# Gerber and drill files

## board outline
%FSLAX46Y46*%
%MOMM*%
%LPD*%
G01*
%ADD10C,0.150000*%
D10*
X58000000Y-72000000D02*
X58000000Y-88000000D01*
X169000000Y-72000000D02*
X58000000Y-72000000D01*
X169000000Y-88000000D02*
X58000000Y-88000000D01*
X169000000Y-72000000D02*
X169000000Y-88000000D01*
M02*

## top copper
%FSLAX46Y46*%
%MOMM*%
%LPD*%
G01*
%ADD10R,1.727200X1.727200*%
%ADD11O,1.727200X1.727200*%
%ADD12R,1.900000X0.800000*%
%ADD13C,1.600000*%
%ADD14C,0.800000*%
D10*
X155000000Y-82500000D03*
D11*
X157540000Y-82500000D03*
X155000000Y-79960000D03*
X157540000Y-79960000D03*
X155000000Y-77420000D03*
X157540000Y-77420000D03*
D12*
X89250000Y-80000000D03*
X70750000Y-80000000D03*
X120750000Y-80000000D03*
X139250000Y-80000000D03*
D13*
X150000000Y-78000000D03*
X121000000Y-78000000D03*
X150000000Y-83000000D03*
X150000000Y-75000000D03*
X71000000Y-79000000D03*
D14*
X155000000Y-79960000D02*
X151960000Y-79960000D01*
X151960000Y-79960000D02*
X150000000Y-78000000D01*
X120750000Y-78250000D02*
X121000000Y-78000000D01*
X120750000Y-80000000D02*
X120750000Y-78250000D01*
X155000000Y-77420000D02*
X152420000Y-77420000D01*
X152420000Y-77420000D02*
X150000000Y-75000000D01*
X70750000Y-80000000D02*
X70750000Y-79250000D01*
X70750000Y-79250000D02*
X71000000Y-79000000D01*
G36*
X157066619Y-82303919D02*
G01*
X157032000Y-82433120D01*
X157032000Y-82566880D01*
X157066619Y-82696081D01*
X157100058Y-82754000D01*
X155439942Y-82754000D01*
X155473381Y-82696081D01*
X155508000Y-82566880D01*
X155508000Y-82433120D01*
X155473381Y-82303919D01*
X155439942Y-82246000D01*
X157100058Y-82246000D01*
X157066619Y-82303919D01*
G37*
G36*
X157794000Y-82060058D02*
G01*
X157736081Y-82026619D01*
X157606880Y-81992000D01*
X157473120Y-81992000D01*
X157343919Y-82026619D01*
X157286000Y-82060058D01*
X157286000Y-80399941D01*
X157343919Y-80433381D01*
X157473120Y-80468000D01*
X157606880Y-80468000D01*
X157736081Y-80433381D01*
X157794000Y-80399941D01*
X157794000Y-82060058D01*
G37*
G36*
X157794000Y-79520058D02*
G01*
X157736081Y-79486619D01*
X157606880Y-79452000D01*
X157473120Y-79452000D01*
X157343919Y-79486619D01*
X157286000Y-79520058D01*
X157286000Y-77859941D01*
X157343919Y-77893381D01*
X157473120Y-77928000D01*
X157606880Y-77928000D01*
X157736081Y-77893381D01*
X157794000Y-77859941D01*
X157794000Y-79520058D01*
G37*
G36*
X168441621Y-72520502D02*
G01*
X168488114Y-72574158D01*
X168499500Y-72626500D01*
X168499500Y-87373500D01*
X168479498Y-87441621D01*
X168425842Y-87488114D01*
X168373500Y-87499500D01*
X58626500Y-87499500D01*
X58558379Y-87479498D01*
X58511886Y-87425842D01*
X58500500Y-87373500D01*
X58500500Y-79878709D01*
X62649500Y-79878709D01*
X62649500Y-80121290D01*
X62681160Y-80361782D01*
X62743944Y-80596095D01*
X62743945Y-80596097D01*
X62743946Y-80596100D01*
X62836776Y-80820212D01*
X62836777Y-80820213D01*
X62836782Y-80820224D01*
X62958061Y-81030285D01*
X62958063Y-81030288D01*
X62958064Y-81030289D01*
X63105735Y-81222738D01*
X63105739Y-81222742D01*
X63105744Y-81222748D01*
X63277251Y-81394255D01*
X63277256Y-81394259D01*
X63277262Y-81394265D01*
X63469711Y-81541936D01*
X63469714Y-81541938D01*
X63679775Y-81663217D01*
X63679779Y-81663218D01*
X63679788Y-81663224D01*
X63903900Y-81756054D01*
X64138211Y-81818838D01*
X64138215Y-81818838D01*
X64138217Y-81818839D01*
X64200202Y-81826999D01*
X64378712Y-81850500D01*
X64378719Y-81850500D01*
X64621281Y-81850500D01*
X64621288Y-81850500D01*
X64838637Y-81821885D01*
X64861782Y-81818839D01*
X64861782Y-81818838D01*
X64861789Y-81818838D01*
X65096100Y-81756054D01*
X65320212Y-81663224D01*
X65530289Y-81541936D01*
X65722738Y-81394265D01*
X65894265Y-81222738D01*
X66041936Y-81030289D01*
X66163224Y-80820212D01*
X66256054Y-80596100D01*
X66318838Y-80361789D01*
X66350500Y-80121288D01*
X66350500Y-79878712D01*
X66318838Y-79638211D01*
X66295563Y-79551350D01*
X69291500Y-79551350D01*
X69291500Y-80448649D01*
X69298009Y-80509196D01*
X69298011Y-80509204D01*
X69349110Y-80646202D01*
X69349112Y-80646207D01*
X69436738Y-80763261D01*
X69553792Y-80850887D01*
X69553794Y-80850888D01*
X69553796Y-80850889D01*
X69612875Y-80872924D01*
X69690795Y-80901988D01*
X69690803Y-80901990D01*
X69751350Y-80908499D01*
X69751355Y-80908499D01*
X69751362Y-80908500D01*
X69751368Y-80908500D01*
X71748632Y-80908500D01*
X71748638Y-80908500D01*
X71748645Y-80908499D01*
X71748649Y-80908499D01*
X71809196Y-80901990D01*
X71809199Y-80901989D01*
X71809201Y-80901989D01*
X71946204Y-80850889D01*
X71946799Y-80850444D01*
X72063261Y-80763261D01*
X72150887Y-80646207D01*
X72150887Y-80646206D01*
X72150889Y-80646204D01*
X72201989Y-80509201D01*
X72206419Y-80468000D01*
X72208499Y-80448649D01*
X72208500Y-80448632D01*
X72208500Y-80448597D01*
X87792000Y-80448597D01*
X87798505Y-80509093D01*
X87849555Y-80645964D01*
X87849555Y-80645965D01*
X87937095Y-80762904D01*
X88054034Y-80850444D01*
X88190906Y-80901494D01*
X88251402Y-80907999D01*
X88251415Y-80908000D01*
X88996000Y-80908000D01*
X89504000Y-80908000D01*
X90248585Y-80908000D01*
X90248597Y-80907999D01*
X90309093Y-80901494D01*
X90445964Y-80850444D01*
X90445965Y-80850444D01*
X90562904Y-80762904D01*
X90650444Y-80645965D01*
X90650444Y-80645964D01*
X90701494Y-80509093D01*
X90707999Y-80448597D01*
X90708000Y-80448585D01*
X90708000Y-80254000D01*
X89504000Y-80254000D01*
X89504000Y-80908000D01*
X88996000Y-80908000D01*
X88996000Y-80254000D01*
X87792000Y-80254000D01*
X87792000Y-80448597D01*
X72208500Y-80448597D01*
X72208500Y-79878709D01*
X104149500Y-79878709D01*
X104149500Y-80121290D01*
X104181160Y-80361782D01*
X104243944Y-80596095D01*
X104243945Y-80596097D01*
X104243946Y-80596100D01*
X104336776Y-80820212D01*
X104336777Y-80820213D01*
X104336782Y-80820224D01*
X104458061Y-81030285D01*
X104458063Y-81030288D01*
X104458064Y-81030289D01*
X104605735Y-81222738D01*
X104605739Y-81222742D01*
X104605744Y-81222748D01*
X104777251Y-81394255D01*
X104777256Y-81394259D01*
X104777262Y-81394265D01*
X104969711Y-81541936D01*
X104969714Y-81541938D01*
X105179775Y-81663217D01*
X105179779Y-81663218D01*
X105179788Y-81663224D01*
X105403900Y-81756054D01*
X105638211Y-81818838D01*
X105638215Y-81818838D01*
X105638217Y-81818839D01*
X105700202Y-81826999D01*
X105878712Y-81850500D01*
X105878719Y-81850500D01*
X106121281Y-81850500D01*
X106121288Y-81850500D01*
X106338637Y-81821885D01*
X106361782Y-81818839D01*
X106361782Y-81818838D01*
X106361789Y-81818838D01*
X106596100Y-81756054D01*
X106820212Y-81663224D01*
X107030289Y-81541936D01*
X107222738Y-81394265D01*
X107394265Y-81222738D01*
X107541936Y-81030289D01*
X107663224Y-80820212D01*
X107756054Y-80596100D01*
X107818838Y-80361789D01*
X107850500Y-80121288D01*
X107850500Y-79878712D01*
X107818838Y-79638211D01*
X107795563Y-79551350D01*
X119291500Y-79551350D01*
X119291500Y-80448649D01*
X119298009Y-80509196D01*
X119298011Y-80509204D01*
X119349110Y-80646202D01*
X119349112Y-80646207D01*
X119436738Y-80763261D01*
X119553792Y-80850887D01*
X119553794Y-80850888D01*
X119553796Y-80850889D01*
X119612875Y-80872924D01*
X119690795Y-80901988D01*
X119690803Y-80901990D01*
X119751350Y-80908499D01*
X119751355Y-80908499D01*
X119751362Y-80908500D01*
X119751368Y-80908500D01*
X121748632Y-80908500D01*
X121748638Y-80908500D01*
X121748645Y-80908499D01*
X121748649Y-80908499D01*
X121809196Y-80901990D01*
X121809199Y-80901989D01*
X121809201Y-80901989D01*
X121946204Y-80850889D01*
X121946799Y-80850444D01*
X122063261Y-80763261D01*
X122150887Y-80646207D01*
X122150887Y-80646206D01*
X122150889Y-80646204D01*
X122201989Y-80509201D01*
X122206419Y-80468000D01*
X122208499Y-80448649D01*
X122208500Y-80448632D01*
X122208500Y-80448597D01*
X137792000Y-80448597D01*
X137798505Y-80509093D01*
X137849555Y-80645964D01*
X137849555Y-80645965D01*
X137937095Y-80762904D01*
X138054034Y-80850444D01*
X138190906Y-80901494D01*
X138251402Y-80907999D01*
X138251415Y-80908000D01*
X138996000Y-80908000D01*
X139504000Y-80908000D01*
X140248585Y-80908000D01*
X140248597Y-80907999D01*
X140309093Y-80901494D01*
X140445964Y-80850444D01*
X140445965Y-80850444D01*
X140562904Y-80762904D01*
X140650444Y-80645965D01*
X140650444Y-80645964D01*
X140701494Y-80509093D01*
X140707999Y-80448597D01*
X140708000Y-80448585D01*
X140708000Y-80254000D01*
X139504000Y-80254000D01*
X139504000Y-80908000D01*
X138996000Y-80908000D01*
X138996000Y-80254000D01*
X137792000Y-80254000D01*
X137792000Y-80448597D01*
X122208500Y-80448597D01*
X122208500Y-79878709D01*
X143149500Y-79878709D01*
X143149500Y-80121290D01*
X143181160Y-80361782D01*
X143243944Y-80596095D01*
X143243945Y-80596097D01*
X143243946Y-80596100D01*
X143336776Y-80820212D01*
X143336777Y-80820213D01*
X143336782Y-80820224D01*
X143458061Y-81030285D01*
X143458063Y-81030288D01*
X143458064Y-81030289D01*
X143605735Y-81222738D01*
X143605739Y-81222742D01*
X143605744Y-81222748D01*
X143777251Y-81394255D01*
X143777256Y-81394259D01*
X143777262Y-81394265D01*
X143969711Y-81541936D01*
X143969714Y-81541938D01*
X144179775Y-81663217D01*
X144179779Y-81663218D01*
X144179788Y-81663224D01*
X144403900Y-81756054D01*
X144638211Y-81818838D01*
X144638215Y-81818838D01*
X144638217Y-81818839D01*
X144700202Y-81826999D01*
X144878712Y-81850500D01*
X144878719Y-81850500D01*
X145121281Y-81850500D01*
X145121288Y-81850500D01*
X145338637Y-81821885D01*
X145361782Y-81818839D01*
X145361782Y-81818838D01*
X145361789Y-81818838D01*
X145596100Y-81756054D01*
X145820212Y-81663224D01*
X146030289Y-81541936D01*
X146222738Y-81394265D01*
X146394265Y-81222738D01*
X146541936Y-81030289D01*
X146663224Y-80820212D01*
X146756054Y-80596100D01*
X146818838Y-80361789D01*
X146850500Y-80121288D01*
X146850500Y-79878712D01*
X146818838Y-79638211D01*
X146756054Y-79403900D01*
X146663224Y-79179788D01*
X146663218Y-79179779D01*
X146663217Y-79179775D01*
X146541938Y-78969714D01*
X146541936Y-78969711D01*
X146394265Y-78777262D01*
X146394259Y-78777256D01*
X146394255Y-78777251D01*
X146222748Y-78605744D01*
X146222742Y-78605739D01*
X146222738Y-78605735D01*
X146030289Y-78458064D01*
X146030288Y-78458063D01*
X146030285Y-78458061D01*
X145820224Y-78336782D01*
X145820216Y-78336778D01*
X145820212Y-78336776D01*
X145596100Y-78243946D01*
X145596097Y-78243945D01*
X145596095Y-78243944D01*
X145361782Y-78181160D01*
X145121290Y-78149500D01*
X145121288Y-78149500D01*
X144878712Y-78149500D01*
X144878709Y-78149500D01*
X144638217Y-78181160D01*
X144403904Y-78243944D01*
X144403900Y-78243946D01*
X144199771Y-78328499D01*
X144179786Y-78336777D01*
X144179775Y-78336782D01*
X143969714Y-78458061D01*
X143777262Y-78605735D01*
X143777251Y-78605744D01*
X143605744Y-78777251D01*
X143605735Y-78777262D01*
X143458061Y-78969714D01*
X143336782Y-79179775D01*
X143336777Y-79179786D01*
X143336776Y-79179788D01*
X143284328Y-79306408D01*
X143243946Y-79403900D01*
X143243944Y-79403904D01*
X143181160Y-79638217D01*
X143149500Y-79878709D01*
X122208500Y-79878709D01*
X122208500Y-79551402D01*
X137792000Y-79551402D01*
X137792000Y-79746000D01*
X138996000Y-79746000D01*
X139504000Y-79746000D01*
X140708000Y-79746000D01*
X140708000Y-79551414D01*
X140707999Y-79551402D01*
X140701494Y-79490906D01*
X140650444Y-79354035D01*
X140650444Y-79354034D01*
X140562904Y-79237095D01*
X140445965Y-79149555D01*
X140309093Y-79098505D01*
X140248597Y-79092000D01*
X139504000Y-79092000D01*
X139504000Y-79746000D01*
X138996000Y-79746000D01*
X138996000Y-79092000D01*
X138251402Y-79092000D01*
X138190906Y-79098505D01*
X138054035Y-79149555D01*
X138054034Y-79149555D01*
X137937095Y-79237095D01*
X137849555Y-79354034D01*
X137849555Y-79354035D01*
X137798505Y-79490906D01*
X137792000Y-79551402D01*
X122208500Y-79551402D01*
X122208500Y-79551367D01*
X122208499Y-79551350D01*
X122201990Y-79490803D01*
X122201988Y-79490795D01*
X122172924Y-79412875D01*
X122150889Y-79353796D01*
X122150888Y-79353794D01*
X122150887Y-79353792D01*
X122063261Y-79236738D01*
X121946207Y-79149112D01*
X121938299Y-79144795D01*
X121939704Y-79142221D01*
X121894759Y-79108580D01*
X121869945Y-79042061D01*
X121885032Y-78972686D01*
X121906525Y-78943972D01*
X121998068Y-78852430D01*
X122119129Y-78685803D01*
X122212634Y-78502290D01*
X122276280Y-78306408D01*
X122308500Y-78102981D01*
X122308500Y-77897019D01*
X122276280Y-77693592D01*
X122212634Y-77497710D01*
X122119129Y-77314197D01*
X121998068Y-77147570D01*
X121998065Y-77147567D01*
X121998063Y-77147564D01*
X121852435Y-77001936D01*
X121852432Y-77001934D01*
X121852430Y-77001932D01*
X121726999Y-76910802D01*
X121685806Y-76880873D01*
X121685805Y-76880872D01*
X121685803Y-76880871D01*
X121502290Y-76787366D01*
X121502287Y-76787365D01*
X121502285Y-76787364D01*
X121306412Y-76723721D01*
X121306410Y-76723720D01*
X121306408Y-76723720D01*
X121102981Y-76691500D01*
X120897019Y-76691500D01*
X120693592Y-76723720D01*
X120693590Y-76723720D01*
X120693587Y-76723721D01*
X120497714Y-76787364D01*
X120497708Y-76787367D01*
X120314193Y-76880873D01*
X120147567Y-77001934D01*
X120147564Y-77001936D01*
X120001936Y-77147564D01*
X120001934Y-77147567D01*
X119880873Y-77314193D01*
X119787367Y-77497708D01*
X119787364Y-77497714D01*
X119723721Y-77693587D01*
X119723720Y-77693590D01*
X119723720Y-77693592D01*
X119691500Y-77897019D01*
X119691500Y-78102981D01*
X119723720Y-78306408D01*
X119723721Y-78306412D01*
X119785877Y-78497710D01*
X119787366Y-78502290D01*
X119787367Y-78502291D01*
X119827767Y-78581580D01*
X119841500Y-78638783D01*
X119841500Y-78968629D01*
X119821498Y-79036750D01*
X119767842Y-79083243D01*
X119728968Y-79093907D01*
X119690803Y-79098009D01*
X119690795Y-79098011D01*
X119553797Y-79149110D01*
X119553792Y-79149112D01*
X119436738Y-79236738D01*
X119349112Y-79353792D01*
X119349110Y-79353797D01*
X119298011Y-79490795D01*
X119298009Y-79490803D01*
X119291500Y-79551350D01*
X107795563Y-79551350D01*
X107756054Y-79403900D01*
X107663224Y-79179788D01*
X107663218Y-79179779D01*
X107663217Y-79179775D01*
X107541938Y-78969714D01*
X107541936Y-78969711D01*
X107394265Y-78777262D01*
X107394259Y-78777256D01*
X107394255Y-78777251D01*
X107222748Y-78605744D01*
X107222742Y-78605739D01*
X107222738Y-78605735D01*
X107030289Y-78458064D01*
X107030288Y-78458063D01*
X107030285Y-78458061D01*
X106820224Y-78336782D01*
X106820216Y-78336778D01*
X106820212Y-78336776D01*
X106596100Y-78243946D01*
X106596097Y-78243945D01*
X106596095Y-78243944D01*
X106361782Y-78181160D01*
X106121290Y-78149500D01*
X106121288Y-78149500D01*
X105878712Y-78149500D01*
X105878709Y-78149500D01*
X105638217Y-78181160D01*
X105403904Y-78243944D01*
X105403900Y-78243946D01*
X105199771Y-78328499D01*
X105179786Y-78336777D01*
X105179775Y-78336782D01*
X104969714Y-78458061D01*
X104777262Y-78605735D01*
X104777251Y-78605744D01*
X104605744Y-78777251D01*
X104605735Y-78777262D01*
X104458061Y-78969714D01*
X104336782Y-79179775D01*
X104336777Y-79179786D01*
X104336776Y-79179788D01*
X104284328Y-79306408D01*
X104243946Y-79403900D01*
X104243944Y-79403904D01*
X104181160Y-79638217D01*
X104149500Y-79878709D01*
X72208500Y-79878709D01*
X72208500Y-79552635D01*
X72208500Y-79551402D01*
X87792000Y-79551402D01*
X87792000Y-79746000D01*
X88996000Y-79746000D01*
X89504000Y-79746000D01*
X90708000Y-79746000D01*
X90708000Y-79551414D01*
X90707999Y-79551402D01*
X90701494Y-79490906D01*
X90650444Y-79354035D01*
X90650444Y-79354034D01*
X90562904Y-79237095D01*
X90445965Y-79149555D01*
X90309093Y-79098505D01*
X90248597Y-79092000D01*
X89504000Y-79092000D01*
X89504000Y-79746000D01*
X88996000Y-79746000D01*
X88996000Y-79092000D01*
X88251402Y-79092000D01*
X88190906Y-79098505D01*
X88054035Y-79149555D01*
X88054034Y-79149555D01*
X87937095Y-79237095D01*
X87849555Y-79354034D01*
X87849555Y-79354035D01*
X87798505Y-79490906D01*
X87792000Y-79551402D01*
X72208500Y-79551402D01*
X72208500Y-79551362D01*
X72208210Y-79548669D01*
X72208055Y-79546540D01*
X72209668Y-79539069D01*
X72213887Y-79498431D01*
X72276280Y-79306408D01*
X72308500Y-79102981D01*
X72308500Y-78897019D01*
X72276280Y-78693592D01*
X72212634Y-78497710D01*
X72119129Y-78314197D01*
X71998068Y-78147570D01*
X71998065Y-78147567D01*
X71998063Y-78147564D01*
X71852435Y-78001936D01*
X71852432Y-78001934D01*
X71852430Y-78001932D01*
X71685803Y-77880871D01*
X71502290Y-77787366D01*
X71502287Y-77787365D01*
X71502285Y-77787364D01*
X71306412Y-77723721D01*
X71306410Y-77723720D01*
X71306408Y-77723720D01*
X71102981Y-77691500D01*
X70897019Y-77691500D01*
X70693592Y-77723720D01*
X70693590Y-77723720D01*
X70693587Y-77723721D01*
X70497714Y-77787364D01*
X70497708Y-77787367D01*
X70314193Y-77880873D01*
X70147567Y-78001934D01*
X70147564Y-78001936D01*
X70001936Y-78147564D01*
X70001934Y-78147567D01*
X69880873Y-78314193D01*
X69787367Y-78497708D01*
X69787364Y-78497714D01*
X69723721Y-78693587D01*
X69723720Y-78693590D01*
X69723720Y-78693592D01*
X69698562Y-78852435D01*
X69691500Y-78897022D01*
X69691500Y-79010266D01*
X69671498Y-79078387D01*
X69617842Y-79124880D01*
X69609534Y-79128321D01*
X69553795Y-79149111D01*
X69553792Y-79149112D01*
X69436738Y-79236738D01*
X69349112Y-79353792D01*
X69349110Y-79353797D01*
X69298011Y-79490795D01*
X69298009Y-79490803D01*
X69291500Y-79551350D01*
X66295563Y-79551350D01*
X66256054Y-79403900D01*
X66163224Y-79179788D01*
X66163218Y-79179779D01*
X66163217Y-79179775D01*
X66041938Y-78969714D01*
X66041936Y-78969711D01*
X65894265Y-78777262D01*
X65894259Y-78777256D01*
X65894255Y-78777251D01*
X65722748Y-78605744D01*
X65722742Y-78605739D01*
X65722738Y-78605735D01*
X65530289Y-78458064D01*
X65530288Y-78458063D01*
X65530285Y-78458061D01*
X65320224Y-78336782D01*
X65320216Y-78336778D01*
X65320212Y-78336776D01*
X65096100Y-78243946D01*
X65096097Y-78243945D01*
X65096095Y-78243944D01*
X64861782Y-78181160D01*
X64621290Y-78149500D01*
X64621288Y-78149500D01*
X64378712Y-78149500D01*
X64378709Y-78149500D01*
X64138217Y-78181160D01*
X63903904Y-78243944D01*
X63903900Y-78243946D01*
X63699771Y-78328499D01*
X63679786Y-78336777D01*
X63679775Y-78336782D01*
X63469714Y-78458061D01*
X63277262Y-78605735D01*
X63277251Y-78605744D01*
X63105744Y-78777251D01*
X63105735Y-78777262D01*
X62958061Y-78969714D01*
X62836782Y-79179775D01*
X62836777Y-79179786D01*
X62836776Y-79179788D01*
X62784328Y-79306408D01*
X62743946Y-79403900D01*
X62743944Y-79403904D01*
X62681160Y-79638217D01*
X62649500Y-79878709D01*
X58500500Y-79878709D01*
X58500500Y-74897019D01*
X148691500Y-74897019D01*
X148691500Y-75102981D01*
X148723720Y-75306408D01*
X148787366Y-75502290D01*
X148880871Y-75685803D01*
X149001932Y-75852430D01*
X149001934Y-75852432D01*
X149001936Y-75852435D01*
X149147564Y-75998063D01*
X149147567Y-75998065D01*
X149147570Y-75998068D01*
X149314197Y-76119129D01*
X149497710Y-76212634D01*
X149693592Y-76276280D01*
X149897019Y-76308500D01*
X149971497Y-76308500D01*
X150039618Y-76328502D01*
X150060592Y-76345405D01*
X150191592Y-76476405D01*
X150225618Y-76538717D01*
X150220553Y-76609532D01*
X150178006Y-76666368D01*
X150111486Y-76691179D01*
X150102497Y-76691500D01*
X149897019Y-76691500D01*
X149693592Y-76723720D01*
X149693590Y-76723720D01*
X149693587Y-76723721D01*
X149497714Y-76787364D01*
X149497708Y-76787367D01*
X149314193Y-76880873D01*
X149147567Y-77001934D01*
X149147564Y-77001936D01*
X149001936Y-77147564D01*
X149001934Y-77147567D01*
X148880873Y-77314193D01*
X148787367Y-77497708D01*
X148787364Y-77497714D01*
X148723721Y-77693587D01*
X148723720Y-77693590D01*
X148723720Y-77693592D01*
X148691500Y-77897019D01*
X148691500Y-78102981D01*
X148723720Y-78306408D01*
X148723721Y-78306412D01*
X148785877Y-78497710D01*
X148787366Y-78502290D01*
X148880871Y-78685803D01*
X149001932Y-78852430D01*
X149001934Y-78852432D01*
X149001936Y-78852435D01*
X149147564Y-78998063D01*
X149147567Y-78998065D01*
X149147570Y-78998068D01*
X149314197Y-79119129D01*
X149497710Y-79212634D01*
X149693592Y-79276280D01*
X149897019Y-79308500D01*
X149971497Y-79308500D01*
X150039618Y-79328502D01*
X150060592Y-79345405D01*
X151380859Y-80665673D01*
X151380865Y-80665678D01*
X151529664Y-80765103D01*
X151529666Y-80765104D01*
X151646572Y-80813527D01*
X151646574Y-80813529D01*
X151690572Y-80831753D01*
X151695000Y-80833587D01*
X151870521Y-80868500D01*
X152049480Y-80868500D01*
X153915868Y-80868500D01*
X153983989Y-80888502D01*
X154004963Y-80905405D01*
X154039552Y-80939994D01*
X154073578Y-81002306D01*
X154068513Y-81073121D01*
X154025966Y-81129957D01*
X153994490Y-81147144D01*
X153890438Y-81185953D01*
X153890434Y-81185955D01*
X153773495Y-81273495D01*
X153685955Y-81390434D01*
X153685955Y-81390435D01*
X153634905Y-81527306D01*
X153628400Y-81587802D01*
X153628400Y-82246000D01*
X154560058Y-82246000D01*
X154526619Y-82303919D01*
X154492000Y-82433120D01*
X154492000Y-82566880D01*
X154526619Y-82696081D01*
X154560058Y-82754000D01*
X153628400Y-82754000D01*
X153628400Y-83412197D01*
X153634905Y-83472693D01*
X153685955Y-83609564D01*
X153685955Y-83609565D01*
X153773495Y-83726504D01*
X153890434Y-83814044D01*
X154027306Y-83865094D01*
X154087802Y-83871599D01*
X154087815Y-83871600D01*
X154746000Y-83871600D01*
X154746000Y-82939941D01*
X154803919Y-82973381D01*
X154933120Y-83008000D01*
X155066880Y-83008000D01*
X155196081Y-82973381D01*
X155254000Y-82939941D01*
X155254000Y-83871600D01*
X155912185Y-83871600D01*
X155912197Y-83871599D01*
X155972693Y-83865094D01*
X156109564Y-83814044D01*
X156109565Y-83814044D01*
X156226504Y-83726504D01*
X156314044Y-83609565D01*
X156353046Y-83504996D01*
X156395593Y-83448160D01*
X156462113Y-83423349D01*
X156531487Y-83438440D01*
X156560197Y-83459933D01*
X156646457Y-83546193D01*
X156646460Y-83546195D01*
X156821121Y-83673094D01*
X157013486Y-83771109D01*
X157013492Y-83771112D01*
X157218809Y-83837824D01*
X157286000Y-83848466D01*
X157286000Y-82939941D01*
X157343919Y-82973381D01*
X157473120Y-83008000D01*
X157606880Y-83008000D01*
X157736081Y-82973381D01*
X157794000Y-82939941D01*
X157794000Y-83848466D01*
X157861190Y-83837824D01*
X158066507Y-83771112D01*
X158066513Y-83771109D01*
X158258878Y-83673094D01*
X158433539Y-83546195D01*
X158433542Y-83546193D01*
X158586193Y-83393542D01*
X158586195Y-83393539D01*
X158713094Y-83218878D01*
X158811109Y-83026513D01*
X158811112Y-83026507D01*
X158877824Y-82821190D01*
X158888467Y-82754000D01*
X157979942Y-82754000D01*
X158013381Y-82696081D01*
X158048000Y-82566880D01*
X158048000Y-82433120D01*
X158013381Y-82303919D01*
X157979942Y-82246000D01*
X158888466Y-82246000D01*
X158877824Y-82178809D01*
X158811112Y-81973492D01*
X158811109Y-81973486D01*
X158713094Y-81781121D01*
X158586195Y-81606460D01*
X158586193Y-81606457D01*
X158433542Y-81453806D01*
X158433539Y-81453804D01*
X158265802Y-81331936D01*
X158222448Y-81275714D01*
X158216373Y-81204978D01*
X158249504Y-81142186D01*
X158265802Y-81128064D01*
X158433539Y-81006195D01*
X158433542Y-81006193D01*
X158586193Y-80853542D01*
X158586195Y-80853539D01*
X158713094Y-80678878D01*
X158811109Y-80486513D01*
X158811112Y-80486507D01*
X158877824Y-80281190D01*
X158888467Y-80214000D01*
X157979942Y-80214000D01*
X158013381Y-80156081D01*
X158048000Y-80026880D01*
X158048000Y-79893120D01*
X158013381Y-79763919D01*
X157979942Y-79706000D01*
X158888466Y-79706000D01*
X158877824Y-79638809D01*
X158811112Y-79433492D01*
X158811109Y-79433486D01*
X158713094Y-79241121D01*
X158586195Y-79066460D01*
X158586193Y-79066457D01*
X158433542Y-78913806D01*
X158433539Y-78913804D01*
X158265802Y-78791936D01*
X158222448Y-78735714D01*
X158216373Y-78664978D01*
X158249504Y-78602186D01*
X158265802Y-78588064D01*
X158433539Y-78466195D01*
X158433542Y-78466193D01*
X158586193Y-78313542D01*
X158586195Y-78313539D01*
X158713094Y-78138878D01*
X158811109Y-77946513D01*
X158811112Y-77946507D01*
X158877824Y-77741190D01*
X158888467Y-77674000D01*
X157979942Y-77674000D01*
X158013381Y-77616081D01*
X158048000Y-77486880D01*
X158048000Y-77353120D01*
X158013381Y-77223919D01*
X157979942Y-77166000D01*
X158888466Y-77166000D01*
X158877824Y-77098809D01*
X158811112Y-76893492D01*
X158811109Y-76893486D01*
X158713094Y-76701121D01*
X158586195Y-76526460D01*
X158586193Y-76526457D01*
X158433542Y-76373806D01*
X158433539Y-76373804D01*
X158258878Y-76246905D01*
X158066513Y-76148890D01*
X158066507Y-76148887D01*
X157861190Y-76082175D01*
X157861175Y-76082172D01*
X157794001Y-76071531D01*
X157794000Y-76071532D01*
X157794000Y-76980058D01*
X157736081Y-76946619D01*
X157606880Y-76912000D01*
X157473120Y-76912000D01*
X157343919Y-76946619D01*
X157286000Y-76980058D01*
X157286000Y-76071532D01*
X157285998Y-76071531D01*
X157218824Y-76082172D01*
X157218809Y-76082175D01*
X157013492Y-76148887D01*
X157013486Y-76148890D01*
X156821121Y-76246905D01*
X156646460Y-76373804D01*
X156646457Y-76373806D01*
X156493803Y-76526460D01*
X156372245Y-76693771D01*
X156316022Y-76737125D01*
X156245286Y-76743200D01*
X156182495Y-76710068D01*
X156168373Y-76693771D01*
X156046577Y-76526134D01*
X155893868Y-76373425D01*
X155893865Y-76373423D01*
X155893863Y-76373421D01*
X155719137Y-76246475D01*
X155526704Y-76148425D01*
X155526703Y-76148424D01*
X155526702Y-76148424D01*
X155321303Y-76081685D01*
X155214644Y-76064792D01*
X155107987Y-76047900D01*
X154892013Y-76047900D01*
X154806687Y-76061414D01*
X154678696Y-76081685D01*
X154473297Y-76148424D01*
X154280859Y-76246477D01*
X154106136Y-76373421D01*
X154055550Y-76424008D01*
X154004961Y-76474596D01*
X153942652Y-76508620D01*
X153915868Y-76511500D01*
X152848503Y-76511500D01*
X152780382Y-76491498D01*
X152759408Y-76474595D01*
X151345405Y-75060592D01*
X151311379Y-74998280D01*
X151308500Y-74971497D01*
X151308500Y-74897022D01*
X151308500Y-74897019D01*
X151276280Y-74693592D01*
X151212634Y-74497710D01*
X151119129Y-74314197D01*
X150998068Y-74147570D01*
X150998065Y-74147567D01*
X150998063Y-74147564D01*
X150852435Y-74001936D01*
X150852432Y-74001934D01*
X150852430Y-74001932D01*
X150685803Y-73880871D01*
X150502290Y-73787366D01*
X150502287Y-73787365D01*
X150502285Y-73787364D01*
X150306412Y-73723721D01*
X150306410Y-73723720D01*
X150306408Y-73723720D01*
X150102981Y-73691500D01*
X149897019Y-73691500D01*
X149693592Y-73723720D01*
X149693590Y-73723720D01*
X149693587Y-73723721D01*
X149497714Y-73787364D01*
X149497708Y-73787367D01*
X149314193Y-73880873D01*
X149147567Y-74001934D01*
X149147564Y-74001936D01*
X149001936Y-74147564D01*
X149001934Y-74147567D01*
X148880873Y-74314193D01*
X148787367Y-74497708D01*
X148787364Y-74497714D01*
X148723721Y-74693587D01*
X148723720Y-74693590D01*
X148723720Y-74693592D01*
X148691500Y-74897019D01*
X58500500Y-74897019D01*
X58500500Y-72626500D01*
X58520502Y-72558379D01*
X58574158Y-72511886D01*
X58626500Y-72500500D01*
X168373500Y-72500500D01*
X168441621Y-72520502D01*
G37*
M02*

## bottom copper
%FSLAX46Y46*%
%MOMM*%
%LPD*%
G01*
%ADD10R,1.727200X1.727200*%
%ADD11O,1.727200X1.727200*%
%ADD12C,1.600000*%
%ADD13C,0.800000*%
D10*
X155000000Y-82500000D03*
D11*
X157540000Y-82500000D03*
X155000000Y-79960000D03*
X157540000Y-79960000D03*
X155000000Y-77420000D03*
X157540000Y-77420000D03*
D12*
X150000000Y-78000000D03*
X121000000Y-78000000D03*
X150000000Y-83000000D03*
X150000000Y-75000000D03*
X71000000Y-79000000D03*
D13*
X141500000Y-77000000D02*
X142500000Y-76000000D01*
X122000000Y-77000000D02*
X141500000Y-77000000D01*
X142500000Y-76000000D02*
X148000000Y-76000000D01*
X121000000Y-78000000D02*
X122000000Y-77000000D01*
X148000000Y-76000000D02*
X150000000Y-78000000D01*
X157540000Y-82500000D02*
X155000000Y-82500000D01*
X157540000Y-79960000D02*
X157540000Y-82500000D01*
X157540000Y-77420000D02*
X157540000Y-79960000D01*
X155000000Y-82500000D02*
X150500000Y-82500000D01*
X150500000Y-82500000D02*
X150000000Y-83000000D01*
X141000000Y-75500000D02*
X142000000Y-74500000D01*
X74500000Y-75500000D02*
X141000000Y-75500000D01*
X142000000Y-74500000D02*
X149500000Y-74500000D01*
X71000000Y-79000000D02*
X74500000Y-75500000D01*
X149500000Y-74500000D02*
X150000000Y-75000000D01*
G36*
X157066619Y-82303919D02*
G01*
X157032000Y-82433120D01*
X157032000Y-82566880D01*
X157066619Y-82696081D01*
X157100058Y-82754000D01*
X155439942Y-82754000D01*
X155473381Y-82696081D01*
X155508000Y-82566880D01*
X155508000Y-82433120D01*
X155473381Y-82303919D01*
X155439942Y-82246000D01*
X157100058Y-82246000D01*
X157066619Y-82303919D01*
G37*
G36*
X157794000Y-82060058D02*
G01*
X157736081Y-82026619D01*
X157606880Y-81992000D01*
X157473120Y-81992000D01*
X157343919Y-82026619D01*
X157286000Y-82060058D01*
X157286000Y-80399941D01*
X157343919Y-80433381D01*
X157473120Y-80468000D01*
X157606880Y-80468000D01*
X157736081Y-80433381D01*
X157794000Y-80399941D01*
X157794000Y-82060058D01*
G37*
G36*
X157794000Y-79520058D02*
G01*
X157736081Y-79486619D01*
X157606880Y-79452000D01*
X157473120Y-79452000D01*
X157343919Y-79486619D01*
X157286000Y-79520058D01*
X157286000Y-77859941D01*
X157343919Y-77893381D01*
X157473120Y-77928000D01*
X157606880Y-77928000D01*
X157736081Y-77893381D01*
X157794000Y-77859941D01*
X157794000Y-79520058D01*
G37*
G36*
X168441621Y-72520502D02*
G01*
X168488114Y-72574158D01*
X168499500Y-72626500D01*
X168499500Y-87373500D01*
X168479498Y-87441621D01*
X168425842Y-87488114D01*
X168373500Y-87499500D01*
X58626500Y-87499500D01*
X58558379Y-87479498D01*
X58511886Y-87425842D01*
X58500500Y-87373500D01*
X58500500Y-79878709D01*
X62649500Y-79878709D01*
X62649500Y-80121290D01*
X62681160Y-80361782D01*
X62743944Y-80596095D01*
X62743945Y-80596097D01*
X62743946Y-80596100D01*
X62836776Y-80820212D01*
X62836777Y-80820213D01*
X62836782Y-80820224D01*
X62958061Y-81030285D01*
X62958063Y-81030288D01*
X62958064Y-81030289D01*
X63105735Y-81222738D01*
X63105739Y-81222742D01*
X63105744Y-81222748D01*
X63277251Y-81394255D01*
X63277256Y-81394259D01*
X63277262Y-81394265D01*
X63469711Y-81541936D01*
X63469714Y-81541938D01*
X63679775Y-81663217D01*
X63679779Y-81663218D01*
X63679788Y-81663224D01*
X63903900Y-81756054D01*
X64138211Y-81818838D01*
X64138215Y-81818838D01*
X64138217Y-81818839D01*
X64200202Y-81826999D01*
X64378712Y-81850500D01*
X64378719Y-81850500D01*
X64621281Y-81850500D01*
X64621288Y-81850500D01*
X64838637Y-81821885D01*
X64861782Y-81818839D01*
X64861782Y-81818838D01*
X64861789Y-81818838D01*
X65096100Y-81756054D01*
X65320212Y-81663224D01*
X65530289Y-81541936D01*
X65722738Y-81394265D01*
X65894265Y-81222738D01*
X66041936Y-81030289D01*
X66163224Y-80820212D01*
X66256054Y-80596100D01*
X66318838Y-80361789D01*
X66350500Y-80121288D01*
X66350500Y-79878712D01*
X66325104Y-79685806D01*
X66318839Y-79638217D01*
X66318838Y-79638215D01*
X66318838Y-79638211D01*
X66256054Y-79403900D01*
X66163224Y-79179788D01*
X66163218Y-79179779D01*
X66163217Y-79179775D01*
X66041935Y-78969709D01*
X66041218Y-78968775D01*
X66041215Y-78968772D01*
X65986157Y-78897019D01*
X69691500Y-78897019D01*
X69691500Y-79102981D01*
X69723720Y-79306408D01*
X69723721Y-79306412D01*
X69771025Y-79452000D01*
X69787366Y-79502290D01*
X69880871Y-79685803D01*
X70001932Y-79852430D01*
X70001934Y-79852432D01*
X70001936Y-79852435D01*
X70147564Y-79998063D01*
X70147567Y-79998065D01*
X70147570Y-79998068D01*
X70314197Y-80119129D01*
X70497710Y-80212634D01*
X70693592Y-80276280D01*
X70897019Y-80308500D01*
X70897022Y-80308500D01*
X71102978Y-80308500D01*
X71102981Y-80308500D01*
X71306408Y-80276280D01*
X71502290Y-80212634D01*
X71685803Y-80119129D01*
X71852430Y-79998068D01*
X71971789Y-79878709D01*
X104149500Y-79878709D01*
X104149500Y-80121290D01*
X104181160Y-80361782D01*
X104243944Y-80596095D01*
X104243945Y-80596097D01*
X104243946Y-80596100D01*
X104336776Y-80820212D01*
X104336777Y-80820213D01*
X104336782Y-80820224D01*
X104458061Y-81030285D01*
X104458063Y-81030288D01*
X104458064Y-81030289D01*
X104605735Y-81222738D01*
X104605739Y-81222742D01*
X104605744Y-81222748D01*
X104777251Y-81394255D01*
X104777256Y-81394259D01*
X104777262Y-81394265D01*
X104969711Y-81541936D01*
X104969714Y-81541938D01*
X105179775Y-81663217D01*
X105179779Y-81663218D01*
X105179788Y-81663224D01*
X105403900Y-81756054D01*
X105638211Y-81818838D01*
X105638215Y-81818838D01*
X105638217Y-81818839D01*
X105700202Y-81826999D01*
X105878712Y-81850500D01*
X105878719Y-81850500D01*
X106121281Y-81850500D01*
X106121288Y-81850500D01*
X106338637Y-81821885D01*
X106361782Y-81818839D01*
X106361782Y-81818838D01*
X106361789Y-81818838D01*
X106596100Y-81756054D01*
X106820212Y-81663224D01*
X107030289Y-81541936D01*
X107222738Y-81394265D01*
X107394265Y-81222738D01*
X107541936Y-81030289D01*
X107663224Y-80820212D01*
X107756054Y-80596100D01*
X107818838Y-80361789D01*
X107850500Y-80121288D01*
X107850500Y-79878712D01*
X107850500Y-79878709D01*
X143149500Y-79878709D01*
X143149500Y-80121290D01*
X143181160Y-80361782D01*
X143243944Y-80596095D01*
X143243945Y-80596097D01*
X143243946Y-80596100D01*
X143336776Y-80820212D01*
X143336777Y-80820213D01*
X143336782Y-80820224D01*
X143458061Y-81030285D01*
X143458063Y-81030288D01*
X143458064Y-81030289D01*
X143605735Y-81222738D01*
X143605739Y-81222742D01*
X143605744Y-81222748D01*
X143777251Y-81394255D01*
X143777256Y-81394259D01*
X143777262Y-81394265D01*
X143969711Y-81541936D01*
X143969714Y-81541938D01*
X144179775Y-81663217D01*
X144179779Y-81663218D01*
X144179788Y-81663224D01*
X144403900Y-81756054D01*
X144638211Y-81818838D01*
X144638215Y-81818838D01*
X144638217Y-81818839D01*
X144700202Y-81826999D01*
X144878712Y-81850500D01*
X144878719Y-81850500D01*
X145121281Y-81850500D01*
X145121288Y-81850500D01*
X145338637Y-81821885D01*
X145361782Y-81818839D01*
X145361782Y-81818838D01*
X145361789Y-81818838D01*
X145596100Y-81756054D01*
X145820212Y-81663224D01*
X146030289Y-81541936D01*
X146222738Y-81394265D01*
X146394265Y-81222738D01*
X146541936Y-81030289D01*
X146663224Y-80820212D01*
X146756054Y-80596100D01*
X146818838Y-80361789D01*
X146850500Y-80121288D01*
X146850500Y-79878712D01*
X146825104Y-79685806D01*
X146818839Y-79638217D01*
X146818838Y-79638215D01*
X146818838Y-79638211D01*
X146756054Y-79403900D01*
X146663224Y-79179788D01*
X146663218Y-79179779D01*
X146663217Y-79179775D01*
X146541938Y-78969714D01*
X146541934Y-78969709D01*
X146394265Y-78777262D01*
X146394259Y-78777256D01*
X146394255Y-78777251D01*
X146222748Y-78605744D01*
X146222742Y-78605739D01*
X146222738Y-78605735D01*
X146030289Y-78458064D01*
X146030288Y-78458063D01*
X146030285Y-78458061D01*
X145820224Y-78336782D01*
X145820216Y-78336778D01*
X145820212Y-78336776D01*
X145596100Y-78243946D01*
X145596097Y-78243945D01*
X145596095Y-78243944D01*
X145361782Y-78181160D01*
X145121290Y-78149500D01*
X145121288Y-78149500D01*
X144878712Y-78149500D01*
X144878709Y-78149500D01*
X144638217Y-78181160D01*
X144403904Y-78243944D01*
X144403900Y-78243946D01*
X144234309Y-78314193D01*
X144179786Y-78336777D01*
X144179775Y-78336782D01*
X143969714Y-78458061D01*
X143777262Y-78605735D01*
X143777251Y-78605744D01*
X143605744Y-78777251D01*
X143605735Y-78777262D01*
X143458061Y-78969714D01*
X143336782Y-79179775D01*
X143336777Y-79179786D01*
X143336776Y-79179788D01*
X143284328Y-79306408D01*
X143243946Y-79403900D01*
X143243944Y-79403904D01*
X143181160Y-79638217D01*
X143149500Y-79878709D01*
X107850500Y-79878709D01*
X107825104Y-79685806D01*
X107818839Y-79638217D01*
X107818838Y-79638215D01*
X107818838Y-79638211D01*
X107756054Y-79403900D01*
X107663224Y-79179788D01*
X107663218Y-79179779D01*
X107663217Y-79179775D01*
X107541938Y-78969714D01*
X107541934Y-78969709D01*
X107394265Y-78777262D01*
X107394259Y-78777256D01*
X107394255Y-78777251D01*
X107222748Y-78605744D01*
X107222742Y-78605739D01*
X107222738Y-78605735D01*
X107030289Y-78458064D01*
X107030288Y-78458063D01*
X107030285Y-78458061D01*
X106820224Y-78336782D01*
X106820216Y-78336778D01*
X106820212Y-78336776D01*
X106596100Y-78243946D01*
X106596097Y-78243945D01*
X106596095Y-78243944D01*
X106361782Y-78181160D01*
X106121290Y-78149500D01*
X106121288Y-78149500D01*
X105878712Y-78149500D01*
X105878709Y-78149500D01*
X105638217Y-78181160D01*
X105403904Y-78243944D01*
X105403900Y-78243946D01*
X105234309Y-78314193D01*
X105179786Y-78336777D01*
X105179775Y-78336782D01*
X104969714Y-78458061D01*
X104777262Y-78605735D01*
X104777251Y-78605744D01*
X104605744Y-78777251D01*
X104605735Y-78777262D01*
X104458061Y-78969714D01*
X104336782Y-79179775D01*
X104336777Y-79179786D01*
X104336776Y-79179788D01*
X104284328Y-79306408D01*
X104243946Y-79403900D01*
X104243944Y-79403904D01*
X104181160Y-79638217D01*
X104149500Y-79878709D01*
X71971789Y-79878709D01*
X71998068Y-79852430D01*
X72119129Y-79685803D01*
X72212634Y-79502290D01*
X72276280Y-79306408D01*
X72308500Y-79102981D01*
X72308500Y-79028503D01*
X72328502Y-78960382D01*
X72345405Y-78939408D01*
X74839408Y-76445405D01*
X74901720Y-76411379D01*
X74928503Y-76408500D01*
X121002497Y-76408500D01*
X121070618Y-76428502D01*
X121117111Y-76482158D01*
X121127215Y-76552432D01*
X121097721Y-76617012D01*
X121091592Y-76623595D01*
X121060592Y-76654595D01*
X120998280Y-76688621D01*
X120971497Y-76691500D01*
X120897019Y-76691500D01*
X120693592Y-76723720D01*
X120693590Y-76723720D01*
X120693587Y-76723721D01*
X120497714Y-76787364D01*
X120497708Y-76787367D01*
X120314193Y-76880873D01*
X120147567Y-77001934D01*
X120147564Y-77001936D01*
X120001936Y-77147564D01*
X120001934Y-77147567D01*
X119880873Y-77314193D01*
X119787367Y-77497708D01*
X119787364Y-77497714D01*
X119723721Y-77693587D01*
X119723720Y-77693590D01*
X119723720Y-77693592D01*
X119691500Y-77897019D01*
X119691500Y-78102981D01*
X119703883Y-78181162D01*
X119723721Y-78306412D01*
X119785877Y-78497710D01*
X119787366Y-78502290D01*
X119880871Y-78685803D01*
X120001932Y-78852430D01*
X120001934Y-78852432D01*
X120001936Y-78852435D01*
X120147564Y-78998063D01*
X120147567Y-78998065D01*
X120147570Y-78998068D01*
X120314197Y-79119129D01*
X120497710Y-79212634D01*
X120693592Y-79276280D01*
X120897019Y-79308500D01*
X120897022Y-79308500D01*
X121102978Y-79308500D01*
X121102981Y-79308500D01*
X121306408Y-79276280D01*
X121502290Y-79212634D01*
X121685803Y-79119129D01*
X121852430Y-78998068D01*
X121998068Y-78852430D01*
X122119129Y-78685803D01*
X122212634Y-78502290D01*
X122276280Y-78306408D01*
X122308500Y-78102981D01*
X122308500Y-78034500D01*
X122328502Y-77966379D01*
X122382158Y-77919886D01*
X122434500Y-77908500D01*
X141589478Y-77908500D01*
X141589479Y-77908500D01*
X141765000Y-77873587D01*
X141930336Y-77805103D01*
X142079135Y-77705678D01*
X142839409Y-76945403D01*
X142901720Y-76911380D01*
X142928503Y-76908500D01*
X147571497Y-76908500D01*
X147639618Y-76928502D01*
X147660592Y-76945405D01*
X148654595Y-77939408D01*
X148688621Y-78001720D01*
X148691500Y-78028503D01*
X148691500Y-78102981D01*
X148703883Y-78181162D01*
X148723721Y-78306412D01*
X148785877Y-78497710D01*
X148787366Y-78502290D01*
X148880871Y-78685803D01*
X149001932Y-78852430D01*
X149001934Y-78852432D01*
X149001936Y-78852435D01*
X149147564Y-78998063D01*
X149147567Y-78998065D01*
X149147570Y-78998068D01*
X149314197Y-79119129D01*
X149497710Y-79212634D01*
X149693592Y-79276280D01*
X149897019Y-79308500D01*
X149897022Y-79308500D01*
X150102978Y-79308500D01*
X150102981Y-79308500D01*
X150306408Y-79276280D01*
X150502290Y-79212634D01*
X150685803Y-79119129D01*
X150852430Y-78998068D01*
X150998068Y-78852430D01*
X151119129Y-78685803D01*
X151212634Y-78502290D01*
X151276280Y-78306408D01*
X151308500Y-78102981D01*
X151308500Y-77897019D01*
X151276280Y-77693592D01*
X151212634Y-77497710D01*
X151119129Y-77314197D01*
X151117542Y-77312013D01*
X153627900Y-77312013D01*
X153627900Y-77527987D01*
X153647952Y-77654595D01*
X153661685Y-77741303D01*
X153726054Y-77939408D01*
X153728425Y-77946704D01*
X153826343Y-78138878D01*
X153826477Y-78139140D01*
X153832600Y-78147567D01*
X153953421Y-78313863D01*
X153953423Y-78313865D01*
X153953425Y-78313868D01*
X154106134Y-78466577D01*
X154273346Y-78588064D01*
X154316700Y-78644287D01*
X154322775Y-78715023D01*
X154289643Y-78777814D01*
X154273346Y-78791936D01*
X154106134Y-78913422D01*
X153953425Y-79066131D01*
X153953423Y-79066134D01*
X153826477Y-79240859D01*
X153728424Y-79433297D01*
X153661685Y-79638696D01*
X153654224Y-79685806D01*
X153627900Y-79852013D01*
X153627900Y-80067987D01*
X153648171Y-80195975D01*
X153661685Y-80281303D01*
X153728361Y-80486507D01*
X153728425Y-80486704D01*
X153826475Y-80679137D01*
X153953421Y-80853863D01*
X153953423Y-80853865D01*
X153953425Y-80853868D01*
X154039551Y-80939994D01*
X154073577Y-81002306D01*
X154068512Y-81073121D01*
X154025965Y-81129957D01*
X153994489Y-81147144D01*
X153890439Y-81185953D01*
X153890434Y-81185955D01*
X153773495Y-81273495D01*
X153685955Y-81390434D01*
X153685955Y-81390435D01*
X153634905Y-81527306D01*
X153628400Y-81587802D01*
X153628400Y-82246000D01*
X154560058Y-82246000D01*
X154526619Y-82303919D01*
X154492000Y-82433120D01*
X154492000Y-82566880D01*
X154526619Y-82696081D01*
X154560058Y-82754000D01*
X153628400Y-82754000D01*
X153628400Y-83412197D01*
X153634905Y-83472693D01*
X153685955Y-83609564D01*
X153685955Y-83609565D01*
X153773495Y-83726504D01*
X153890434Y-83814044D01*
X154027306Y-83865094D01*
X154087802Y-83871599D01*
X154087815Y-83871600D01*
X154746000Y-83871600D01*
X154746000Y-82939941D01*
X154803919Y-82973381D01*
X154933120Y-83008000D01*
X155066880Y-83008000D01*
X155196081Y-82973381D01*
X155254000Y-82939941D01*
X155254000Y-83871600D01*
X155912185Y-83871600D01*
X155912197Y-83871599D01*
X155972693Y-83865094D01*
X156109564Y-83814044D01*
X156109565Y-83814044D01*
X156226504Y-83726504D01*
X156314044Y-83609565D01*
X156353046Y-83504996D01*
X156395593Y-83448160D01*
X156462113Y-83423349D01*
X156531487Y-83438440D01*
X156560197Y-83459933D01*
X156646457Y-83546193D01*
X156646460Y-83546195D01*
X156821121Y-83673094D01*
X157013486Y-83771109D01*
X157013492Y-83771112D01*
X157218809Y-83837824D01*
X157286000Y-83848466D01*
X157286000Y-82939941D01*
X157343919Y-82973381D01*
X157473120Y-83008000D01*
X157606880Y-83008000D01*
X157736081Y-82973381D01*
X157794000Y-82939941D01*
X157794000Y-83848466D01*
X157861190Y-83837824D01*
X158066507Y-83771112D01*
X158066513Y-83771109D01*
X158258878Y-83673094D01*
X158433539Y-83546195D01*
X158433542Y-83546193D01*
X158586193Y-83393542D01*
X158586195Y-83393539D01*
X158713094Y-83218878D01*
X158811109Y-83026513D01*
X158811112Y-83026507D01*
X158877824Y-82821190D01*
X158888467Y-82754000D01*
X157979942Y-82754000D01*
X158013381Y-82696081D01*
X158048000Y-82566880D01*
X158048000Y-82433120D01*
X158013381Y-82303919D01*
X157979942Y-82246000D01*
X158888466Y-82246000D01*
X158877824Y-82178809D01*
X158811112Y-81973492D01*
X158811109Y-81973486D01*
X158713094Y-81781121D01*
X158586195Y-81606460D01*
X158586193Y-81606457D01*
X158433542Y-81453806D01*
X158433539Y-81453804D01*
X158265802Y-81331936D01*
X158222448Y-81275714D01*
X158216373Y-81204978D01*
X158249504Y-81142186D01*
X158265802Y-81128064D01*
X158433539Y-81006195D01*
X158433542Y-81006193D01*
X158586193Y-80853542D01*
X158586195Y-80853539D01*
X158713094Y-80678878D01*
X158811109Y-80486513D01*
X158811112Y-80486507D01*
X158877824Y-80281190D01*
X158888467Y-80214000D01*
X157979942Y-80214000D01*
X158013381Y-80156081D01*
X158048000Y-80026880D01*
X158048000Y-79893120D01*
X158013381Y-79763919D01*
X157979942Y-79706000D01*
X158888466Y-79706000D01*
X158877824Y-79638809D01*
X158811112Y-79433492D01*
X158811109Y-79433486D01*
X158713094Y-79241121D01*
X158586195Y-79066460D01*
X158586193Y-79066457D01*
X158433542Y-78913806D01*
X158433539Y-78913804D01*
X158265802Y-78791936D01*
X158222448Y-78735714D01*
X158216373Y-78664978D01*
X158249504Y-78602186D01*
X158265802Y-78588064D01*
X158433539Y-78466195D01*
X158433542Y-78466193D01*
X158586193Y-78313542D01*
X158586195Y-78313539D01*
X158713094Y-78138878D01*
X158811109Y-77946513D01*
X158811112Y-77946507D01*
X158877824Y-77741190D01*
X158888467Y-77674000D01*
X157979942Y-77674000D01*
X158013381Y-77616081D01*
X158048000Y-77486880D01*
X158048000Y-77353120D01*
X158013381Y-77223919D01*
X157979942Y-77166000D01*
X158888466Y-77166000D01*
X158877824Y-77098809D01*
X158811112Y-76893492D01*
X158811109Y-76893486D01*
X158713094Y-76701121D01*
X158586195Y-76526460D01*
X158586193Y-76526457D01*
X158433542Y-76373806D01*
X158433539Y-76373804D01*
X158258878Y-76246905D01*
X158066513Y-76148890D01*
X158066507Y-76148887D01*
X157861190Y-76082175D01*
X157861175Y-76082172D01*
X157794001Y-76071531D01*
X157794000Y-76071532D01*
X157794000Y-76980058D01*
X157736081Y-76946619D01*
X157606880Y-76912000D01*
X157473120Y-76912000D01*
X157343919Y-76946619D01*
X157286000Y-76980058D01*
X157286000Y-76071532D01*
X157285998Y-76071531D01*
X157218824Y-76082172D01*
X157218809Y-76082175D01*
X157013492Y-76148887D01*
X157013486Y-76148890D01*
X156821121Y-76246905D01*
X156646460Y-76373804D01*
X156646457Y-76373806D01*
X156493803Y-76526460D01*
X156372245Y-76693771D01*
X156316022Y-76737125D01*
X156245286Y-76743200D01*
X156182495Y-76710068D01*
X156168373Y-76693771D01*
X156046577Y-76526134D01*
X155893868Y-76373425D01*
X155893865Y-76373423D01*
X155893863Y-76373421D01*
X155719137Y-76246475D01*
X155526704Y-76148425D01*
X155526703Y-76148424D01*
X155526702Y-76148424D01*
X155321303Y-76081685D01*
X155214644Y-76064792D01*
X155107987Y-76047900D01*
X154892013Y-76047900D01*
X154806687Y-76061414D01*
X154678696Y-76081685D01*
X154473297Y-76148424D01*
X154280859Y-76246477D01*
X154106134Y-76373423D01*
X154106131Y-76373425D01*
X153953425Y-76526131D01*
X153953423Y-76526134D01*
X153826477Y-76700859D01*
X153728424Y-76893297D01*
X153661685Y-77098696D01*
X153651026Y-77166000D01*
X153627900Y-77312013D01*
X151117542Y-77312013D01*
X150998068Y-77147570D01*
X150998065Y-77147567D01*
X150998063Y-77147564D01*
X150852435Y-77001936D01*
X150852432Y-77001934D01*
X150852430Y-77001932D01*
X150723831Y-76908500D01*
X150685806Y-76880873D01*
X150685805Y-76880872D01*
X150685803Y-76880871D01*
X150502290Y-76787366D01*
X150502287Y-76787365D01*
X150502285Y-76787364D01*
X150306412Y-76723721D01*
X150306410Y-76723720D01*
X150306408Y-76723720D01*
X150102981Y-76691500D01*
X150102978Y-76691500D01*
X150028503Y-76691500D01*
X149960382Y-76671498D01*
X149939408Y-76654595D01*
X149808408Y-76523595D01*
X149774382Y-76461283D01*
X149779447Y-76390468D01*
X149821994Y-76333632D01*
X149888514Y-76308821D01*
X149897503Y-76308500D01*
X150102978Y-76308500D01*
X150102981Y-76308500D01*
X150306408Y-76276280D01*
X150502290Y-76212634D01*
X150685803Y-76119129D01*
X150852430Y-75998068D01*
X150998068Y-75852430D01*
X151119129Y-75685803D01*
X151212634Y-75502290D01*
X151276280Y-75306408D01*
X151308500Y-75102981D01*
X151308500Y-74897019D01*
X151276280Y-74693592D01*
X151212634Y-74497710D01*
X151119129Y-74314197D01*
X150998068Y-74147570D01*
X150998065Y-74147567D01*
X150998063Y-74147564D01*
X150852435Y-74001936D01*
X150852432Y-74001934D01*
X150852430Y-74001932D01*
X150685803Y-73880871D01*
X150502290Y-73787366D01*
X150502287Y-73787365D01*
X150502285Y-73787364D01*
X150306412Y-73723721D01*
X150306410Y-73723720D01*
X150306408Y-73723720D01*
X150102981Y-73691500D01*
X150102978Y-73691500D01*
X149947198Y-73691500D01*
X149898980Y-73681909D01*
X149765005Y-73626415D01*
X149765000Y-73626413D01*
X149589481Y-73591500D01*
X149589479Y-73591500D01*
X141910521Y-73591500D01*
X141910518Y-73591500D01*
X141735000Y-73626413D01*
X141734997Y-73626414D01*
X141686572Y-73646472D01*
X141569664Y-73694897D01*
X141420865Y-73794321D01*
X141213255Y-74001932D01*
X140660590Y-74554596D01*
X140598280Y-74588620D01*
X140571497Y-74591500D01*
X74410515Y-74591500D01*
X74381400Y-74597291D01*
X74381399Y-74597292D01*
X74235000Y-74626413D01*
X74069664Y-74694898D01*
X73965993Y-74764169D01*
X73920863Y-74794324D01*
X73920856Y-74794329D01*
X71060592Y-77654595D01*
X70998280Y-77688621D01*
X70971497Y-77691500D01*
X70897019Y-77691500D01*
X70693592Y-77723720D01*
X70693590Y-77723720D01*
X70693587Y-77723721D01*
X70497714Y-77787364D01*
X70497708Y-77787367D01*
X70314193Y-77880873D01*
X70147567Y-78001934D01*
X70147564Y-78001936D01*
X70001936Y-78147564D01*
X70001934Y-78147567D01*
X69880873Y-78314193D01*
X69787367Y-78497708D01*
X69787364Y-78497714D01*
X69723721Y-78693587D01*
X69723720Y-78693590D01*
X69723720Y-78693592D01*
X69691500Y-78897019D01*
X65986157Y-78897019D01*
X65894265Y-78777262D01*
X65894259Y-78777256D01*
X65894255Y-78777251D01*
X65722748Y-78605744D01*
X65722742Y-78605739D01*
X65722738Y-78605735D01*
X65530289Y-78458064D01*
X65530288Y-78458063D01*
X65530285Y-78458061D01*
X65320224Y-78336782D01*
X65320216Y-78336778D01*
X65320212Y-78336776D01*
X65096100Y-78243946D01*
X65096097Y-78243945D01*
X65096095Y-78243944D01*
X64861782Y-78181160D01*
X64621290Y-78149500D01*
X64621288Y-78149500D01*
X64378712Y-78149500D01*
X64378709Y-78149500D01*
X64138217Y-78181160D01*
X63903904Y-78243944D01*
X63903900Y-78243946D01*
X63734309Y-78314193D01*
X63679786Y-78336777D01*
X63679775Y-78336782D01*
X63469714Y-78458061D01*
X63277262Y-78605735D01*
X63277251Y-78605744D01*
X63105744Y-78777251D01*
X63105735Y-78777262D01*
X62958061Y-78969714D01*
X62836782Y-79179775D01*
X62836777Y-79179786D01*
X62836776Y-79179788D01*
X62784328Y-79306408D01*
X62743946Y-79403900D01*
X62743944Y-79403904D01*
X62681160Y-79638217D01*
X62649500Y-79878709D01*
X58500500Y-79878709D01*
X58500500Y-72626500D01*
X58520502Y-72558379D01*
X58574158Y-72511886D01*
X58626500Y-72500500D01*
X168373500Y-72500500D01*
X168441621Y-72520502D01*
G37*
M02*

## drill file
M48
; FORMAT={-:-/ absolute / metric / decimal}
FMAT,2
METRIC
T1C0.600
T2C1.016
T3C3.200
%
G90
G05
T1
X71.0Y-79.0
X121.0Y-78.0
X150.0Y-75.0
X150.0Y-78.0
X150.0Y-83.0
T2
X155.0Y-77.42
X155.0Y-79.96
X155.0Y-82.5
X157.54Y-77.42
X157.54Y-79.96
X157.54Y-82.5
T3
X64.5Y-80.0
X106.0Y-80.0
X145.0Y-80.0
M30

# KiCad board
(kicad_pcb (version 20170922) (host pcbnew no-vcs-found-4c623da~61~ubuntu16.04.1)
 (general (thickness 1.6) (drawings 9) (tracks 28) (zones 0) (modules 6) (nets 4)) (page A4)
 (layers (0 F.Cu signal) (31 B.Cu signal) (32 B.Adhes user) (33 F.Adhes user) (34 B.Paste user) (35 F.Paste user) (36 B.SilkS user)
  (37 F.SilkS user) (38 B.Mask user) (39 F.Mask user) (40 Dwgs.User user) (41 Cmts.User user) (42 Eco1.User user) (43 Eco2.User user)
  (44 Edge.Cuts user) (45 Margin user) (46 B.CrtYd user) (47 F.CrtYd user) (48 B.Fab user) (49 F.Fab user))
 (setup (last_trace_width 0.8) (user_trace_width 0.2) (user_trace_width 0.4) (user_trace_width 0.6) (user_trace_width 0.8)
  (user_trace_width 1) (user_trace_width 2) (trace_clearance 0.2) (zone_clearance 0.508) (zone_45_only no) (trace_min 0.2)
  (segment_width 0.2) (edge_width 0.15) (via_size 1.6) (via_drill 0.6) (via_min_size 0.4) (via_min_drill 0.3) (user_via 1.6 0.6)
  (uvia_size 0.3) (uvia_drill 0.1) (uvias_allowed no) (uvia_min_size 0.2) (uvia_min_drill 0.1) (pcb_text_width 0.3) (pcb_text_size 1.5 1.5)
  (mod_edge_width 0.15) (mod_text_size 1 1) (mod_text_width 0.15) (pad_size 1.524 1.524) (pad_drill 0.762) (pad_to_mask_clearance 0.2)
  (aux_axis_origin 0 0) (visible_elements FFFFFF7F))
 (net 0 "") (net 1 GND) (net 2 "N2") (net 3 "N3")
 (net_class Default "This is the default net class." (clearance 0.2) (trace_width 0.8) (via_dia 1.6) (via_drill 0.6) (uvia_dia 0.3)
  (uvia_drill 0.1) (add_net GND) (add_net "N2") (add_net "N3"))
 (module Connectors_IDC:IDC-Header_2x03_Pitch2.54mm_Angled (layer B.Cu) (at 155 82.5)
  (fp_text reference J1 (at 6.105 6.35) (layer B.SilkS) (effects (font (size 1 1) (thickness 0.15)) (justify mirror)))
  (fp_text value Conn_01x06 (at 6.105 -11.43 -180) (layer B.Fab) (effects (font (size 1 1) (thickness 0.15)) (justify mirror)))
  (pad 1 thru_hole rect (at 0 0) (size 1.7272 1.7272) (drill 1.016) (layers *.Cu *.Mask) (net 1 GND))
  (pad 2 thru_hole oval (at 2.54 0) (size 1.7272 1.7272) (drill 1.016) (layers *.Cu *.Mask) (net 1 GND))
  (pad 3 thru_hole oval (at 0 -2.54) (size 1.7272 1.7272) (drill 1.016) (layers *.Cu *.Mask) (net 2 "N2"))
  (pad 4 thru_hole oval (at 2.54 -2.54) (size 1.7272 1.7272) (drill 1.016) (layers *.Cu *.Mask) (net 1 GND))
  (pad 5 thru_hole oval (at 0 -5.08) (size 1.7272 1.7272) (drill 1.016) (layers *.Cu *.Mask) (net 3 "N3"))
  (pad 6 thru_hole oval (at 2.54 -5.08) (size 1.7272 1.7272) (drill 1.016) (layers *.Cu *.Mask) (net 1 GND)))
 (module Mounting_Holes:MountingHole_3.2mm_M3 (layer F.Cu) (at 145 80)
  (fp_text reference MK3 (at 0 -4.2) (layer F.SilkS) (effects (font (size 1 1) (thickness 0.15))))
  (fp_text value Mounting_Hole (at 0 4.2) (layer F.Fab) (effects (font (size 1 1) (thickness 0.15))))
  (pad 1 np_thru_hole circle (at 0 0) (size 3.2 3.2) (drill 3.2) (layers *.Cu *.Mask)))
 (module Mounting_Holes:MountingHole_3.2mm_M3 (layer F.Cu) (at 106 80)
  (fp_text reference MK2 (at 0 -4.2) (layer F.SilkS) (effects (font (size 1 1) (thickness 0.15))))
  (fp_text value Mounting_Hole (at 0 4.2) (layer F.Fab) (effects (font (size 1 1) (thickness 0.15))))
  (pad 1 np_thru_hole circle (at 0 0) (size 3.2 3.2) (drill 3.2) (layers *.Cu *.Mask)))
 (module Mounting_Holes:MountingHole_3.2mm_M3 (layer F.Cu) (at 64.5 80)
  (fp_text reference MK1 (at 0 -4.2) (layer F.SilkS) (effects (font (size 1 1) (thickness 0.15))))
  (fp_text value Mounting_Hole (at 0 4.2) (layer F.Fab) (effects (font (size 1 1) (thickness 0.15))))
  (pad 1 np_thru_hole circle (at 0 0) (size 3.2 3.2) (drill 3.2) (layers *.Cu *.Mask)))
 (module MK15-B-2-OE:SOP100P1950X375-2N (layer F.Cu) (at 80 80)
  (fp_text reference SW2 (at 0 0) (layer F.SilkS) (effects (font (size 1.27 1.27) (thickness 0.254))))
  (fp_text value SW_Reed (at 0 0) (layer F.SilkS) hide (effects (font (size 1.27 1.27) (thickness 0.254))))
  (pad 2 smd rect (at 9.25 0 90) (size 0.8 1.9) (layers F.Cu F.Paste F.Mask) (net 1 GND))
  (pad 1 smd rect (at -9.25 0 90) (size 0.8 1.9) (layers F.Cu F.Paste F.Mask) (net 3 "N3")))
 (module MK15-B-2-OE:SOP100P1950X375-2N (layer F.Cu) (at 130 80)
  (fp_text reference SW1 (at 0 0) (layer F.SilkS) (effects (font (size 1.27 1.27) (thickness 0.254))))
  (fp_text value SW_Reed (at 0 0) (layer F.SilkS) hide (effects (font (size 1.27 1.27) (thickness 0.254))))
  (pad 1 smd rect (at -9.25 0 90) (size 0.8 1.9) (layers F.Cu F.Paste F.Mask) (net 2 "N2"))
  (pad 2 smd rect (at 9.25 0 90) (size 0.8 1.9) (layers F.Cu F.Paste F.Mask) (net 1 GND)))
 (gr_line (start 58 72) (end 58 88) (layer Edge.Cuts) (width 0.15))
 (gr_line (start 169 72) (end 58 72) (layer Edge.Cuts) (width 0.15))
 (gr_line (start 169 88) (end 58 88) (layer Edge.Cuts) (width 0.15))
 (gr_line (start 169 72) (end 169 88) (layer Edge.Cuts) (width 0.15))
 (segment (start 141.5 77) (end 142.5 76) (width 0.8) (layer B.Cu) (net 2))
 (segment (start 122 77) (end 141.5 77) (width 0.8) (layer B.Cu) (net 2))
 (segment (start 142.5 76) (end 148 76) (width 0.8) (layer B.Cu) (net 2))
 (segment (start 121 78) (end 122 77) (width 0.8) (layer B.Cu) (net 2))
 (segment (start 148 76) (end 150 78) (width 0.8) (layer B.Cu) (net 2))
 (segment (start 155 79.96) (end 151.96 79.96) (width 0.8) (layer F.Cu) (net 2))
 (segment (start 151.96 79.96) (end 150 78) (width 0.8) (layer F.Cu) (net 2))
 (via (at 150 78) (size 1.6) (drill 0.6) (layers F.Cu B.Cu) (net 2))
 (segment (start 120.75 78.25) (end 121 78) (width 0.8) (layer F.Cu) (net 2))
 (segment (start 120.75 80) (end 120.75 78.25) (width 0.8) (layer F.Cu) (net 2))
 (via (at 121 78) (size 1.6) (drill 0.6) (layers F.Cu B.Cu) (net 2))
 (segment (start 157.54 82.5) (end 155 82.5) (width 0.8) (layer B.Cu) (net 1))
 (segment (start 157.54 79.96) (end 157.54 82.5) (width 0.8) (layer B.Cu) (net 1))
 (segment (start 157.54 77.42) (end 157.54 79.96) (width 0.8) (layer B.Cu) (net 1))
 (segment (start 155 82.5) (end 150.5 82.5) (width 0.8) (layer B.Cu) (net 1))
 (segment (start 150.5 82.5) (end 150 83) (width 0.8) (layer B.Cu) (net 1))
 (via (at 150 83) (size 1.6) (drill 0.6) (layers F.Cu B.Cu) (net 1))
 (segment (start 141 75.5) (end 142 74.5) (width 0.8) (layer B.Cu) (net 3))
 (segment (start 74.5 75.5) (end 141 75.5) (width 0.8) (layer B.Cu) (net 3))
 (segment (start 142 74.5) (end 149.5 74.5) (width 0.8) (layer B.Cu) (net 3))
 (segment (start 71 79) (end 74.5 75.5) (width 0.8) (layer B.Cu) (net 3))
 (segment (start 149.5 74.5) (end 150 75) (width 0.8) (layer B.Cu) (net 3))
 (segment (start 155 77.42) (end 152.42 77.42) (width 0.8) (layer F.Cu) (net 3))
 (segment (start 152.42 77.42) (end 150 75) (width 0.8) (layer F.Cu) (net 3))
 (via (at 150 75) (size 1.6) (drill 0.6) (layers F.Cu B.Cu) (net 3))
 (segment (start 70.75 80) (end 70.75 79.25) (width 0.8) (layer F.Cu) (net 3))
 (segment (start 70.75 79.25) (end 71 79) (width 0.8) (layer F.Cu) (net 3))
 (via (at 71 79) (size 1.6) (drill 0.6) (layers F.Cu B.Cu) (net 3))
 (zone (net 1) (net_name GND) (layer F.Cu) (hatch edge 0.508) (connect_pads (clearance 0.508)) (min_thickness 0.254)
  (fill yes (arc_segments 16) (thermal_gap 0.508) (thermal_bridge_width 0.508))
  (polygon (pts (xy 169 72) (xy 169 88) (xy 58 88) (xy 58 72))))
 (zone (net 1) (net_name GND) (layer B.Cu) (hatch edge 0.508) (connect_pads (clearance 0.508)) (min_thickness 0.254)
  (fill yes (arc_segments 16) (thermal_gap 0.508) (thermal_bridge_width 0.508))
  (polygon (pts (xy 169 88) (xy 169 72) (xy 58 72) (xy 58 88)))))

